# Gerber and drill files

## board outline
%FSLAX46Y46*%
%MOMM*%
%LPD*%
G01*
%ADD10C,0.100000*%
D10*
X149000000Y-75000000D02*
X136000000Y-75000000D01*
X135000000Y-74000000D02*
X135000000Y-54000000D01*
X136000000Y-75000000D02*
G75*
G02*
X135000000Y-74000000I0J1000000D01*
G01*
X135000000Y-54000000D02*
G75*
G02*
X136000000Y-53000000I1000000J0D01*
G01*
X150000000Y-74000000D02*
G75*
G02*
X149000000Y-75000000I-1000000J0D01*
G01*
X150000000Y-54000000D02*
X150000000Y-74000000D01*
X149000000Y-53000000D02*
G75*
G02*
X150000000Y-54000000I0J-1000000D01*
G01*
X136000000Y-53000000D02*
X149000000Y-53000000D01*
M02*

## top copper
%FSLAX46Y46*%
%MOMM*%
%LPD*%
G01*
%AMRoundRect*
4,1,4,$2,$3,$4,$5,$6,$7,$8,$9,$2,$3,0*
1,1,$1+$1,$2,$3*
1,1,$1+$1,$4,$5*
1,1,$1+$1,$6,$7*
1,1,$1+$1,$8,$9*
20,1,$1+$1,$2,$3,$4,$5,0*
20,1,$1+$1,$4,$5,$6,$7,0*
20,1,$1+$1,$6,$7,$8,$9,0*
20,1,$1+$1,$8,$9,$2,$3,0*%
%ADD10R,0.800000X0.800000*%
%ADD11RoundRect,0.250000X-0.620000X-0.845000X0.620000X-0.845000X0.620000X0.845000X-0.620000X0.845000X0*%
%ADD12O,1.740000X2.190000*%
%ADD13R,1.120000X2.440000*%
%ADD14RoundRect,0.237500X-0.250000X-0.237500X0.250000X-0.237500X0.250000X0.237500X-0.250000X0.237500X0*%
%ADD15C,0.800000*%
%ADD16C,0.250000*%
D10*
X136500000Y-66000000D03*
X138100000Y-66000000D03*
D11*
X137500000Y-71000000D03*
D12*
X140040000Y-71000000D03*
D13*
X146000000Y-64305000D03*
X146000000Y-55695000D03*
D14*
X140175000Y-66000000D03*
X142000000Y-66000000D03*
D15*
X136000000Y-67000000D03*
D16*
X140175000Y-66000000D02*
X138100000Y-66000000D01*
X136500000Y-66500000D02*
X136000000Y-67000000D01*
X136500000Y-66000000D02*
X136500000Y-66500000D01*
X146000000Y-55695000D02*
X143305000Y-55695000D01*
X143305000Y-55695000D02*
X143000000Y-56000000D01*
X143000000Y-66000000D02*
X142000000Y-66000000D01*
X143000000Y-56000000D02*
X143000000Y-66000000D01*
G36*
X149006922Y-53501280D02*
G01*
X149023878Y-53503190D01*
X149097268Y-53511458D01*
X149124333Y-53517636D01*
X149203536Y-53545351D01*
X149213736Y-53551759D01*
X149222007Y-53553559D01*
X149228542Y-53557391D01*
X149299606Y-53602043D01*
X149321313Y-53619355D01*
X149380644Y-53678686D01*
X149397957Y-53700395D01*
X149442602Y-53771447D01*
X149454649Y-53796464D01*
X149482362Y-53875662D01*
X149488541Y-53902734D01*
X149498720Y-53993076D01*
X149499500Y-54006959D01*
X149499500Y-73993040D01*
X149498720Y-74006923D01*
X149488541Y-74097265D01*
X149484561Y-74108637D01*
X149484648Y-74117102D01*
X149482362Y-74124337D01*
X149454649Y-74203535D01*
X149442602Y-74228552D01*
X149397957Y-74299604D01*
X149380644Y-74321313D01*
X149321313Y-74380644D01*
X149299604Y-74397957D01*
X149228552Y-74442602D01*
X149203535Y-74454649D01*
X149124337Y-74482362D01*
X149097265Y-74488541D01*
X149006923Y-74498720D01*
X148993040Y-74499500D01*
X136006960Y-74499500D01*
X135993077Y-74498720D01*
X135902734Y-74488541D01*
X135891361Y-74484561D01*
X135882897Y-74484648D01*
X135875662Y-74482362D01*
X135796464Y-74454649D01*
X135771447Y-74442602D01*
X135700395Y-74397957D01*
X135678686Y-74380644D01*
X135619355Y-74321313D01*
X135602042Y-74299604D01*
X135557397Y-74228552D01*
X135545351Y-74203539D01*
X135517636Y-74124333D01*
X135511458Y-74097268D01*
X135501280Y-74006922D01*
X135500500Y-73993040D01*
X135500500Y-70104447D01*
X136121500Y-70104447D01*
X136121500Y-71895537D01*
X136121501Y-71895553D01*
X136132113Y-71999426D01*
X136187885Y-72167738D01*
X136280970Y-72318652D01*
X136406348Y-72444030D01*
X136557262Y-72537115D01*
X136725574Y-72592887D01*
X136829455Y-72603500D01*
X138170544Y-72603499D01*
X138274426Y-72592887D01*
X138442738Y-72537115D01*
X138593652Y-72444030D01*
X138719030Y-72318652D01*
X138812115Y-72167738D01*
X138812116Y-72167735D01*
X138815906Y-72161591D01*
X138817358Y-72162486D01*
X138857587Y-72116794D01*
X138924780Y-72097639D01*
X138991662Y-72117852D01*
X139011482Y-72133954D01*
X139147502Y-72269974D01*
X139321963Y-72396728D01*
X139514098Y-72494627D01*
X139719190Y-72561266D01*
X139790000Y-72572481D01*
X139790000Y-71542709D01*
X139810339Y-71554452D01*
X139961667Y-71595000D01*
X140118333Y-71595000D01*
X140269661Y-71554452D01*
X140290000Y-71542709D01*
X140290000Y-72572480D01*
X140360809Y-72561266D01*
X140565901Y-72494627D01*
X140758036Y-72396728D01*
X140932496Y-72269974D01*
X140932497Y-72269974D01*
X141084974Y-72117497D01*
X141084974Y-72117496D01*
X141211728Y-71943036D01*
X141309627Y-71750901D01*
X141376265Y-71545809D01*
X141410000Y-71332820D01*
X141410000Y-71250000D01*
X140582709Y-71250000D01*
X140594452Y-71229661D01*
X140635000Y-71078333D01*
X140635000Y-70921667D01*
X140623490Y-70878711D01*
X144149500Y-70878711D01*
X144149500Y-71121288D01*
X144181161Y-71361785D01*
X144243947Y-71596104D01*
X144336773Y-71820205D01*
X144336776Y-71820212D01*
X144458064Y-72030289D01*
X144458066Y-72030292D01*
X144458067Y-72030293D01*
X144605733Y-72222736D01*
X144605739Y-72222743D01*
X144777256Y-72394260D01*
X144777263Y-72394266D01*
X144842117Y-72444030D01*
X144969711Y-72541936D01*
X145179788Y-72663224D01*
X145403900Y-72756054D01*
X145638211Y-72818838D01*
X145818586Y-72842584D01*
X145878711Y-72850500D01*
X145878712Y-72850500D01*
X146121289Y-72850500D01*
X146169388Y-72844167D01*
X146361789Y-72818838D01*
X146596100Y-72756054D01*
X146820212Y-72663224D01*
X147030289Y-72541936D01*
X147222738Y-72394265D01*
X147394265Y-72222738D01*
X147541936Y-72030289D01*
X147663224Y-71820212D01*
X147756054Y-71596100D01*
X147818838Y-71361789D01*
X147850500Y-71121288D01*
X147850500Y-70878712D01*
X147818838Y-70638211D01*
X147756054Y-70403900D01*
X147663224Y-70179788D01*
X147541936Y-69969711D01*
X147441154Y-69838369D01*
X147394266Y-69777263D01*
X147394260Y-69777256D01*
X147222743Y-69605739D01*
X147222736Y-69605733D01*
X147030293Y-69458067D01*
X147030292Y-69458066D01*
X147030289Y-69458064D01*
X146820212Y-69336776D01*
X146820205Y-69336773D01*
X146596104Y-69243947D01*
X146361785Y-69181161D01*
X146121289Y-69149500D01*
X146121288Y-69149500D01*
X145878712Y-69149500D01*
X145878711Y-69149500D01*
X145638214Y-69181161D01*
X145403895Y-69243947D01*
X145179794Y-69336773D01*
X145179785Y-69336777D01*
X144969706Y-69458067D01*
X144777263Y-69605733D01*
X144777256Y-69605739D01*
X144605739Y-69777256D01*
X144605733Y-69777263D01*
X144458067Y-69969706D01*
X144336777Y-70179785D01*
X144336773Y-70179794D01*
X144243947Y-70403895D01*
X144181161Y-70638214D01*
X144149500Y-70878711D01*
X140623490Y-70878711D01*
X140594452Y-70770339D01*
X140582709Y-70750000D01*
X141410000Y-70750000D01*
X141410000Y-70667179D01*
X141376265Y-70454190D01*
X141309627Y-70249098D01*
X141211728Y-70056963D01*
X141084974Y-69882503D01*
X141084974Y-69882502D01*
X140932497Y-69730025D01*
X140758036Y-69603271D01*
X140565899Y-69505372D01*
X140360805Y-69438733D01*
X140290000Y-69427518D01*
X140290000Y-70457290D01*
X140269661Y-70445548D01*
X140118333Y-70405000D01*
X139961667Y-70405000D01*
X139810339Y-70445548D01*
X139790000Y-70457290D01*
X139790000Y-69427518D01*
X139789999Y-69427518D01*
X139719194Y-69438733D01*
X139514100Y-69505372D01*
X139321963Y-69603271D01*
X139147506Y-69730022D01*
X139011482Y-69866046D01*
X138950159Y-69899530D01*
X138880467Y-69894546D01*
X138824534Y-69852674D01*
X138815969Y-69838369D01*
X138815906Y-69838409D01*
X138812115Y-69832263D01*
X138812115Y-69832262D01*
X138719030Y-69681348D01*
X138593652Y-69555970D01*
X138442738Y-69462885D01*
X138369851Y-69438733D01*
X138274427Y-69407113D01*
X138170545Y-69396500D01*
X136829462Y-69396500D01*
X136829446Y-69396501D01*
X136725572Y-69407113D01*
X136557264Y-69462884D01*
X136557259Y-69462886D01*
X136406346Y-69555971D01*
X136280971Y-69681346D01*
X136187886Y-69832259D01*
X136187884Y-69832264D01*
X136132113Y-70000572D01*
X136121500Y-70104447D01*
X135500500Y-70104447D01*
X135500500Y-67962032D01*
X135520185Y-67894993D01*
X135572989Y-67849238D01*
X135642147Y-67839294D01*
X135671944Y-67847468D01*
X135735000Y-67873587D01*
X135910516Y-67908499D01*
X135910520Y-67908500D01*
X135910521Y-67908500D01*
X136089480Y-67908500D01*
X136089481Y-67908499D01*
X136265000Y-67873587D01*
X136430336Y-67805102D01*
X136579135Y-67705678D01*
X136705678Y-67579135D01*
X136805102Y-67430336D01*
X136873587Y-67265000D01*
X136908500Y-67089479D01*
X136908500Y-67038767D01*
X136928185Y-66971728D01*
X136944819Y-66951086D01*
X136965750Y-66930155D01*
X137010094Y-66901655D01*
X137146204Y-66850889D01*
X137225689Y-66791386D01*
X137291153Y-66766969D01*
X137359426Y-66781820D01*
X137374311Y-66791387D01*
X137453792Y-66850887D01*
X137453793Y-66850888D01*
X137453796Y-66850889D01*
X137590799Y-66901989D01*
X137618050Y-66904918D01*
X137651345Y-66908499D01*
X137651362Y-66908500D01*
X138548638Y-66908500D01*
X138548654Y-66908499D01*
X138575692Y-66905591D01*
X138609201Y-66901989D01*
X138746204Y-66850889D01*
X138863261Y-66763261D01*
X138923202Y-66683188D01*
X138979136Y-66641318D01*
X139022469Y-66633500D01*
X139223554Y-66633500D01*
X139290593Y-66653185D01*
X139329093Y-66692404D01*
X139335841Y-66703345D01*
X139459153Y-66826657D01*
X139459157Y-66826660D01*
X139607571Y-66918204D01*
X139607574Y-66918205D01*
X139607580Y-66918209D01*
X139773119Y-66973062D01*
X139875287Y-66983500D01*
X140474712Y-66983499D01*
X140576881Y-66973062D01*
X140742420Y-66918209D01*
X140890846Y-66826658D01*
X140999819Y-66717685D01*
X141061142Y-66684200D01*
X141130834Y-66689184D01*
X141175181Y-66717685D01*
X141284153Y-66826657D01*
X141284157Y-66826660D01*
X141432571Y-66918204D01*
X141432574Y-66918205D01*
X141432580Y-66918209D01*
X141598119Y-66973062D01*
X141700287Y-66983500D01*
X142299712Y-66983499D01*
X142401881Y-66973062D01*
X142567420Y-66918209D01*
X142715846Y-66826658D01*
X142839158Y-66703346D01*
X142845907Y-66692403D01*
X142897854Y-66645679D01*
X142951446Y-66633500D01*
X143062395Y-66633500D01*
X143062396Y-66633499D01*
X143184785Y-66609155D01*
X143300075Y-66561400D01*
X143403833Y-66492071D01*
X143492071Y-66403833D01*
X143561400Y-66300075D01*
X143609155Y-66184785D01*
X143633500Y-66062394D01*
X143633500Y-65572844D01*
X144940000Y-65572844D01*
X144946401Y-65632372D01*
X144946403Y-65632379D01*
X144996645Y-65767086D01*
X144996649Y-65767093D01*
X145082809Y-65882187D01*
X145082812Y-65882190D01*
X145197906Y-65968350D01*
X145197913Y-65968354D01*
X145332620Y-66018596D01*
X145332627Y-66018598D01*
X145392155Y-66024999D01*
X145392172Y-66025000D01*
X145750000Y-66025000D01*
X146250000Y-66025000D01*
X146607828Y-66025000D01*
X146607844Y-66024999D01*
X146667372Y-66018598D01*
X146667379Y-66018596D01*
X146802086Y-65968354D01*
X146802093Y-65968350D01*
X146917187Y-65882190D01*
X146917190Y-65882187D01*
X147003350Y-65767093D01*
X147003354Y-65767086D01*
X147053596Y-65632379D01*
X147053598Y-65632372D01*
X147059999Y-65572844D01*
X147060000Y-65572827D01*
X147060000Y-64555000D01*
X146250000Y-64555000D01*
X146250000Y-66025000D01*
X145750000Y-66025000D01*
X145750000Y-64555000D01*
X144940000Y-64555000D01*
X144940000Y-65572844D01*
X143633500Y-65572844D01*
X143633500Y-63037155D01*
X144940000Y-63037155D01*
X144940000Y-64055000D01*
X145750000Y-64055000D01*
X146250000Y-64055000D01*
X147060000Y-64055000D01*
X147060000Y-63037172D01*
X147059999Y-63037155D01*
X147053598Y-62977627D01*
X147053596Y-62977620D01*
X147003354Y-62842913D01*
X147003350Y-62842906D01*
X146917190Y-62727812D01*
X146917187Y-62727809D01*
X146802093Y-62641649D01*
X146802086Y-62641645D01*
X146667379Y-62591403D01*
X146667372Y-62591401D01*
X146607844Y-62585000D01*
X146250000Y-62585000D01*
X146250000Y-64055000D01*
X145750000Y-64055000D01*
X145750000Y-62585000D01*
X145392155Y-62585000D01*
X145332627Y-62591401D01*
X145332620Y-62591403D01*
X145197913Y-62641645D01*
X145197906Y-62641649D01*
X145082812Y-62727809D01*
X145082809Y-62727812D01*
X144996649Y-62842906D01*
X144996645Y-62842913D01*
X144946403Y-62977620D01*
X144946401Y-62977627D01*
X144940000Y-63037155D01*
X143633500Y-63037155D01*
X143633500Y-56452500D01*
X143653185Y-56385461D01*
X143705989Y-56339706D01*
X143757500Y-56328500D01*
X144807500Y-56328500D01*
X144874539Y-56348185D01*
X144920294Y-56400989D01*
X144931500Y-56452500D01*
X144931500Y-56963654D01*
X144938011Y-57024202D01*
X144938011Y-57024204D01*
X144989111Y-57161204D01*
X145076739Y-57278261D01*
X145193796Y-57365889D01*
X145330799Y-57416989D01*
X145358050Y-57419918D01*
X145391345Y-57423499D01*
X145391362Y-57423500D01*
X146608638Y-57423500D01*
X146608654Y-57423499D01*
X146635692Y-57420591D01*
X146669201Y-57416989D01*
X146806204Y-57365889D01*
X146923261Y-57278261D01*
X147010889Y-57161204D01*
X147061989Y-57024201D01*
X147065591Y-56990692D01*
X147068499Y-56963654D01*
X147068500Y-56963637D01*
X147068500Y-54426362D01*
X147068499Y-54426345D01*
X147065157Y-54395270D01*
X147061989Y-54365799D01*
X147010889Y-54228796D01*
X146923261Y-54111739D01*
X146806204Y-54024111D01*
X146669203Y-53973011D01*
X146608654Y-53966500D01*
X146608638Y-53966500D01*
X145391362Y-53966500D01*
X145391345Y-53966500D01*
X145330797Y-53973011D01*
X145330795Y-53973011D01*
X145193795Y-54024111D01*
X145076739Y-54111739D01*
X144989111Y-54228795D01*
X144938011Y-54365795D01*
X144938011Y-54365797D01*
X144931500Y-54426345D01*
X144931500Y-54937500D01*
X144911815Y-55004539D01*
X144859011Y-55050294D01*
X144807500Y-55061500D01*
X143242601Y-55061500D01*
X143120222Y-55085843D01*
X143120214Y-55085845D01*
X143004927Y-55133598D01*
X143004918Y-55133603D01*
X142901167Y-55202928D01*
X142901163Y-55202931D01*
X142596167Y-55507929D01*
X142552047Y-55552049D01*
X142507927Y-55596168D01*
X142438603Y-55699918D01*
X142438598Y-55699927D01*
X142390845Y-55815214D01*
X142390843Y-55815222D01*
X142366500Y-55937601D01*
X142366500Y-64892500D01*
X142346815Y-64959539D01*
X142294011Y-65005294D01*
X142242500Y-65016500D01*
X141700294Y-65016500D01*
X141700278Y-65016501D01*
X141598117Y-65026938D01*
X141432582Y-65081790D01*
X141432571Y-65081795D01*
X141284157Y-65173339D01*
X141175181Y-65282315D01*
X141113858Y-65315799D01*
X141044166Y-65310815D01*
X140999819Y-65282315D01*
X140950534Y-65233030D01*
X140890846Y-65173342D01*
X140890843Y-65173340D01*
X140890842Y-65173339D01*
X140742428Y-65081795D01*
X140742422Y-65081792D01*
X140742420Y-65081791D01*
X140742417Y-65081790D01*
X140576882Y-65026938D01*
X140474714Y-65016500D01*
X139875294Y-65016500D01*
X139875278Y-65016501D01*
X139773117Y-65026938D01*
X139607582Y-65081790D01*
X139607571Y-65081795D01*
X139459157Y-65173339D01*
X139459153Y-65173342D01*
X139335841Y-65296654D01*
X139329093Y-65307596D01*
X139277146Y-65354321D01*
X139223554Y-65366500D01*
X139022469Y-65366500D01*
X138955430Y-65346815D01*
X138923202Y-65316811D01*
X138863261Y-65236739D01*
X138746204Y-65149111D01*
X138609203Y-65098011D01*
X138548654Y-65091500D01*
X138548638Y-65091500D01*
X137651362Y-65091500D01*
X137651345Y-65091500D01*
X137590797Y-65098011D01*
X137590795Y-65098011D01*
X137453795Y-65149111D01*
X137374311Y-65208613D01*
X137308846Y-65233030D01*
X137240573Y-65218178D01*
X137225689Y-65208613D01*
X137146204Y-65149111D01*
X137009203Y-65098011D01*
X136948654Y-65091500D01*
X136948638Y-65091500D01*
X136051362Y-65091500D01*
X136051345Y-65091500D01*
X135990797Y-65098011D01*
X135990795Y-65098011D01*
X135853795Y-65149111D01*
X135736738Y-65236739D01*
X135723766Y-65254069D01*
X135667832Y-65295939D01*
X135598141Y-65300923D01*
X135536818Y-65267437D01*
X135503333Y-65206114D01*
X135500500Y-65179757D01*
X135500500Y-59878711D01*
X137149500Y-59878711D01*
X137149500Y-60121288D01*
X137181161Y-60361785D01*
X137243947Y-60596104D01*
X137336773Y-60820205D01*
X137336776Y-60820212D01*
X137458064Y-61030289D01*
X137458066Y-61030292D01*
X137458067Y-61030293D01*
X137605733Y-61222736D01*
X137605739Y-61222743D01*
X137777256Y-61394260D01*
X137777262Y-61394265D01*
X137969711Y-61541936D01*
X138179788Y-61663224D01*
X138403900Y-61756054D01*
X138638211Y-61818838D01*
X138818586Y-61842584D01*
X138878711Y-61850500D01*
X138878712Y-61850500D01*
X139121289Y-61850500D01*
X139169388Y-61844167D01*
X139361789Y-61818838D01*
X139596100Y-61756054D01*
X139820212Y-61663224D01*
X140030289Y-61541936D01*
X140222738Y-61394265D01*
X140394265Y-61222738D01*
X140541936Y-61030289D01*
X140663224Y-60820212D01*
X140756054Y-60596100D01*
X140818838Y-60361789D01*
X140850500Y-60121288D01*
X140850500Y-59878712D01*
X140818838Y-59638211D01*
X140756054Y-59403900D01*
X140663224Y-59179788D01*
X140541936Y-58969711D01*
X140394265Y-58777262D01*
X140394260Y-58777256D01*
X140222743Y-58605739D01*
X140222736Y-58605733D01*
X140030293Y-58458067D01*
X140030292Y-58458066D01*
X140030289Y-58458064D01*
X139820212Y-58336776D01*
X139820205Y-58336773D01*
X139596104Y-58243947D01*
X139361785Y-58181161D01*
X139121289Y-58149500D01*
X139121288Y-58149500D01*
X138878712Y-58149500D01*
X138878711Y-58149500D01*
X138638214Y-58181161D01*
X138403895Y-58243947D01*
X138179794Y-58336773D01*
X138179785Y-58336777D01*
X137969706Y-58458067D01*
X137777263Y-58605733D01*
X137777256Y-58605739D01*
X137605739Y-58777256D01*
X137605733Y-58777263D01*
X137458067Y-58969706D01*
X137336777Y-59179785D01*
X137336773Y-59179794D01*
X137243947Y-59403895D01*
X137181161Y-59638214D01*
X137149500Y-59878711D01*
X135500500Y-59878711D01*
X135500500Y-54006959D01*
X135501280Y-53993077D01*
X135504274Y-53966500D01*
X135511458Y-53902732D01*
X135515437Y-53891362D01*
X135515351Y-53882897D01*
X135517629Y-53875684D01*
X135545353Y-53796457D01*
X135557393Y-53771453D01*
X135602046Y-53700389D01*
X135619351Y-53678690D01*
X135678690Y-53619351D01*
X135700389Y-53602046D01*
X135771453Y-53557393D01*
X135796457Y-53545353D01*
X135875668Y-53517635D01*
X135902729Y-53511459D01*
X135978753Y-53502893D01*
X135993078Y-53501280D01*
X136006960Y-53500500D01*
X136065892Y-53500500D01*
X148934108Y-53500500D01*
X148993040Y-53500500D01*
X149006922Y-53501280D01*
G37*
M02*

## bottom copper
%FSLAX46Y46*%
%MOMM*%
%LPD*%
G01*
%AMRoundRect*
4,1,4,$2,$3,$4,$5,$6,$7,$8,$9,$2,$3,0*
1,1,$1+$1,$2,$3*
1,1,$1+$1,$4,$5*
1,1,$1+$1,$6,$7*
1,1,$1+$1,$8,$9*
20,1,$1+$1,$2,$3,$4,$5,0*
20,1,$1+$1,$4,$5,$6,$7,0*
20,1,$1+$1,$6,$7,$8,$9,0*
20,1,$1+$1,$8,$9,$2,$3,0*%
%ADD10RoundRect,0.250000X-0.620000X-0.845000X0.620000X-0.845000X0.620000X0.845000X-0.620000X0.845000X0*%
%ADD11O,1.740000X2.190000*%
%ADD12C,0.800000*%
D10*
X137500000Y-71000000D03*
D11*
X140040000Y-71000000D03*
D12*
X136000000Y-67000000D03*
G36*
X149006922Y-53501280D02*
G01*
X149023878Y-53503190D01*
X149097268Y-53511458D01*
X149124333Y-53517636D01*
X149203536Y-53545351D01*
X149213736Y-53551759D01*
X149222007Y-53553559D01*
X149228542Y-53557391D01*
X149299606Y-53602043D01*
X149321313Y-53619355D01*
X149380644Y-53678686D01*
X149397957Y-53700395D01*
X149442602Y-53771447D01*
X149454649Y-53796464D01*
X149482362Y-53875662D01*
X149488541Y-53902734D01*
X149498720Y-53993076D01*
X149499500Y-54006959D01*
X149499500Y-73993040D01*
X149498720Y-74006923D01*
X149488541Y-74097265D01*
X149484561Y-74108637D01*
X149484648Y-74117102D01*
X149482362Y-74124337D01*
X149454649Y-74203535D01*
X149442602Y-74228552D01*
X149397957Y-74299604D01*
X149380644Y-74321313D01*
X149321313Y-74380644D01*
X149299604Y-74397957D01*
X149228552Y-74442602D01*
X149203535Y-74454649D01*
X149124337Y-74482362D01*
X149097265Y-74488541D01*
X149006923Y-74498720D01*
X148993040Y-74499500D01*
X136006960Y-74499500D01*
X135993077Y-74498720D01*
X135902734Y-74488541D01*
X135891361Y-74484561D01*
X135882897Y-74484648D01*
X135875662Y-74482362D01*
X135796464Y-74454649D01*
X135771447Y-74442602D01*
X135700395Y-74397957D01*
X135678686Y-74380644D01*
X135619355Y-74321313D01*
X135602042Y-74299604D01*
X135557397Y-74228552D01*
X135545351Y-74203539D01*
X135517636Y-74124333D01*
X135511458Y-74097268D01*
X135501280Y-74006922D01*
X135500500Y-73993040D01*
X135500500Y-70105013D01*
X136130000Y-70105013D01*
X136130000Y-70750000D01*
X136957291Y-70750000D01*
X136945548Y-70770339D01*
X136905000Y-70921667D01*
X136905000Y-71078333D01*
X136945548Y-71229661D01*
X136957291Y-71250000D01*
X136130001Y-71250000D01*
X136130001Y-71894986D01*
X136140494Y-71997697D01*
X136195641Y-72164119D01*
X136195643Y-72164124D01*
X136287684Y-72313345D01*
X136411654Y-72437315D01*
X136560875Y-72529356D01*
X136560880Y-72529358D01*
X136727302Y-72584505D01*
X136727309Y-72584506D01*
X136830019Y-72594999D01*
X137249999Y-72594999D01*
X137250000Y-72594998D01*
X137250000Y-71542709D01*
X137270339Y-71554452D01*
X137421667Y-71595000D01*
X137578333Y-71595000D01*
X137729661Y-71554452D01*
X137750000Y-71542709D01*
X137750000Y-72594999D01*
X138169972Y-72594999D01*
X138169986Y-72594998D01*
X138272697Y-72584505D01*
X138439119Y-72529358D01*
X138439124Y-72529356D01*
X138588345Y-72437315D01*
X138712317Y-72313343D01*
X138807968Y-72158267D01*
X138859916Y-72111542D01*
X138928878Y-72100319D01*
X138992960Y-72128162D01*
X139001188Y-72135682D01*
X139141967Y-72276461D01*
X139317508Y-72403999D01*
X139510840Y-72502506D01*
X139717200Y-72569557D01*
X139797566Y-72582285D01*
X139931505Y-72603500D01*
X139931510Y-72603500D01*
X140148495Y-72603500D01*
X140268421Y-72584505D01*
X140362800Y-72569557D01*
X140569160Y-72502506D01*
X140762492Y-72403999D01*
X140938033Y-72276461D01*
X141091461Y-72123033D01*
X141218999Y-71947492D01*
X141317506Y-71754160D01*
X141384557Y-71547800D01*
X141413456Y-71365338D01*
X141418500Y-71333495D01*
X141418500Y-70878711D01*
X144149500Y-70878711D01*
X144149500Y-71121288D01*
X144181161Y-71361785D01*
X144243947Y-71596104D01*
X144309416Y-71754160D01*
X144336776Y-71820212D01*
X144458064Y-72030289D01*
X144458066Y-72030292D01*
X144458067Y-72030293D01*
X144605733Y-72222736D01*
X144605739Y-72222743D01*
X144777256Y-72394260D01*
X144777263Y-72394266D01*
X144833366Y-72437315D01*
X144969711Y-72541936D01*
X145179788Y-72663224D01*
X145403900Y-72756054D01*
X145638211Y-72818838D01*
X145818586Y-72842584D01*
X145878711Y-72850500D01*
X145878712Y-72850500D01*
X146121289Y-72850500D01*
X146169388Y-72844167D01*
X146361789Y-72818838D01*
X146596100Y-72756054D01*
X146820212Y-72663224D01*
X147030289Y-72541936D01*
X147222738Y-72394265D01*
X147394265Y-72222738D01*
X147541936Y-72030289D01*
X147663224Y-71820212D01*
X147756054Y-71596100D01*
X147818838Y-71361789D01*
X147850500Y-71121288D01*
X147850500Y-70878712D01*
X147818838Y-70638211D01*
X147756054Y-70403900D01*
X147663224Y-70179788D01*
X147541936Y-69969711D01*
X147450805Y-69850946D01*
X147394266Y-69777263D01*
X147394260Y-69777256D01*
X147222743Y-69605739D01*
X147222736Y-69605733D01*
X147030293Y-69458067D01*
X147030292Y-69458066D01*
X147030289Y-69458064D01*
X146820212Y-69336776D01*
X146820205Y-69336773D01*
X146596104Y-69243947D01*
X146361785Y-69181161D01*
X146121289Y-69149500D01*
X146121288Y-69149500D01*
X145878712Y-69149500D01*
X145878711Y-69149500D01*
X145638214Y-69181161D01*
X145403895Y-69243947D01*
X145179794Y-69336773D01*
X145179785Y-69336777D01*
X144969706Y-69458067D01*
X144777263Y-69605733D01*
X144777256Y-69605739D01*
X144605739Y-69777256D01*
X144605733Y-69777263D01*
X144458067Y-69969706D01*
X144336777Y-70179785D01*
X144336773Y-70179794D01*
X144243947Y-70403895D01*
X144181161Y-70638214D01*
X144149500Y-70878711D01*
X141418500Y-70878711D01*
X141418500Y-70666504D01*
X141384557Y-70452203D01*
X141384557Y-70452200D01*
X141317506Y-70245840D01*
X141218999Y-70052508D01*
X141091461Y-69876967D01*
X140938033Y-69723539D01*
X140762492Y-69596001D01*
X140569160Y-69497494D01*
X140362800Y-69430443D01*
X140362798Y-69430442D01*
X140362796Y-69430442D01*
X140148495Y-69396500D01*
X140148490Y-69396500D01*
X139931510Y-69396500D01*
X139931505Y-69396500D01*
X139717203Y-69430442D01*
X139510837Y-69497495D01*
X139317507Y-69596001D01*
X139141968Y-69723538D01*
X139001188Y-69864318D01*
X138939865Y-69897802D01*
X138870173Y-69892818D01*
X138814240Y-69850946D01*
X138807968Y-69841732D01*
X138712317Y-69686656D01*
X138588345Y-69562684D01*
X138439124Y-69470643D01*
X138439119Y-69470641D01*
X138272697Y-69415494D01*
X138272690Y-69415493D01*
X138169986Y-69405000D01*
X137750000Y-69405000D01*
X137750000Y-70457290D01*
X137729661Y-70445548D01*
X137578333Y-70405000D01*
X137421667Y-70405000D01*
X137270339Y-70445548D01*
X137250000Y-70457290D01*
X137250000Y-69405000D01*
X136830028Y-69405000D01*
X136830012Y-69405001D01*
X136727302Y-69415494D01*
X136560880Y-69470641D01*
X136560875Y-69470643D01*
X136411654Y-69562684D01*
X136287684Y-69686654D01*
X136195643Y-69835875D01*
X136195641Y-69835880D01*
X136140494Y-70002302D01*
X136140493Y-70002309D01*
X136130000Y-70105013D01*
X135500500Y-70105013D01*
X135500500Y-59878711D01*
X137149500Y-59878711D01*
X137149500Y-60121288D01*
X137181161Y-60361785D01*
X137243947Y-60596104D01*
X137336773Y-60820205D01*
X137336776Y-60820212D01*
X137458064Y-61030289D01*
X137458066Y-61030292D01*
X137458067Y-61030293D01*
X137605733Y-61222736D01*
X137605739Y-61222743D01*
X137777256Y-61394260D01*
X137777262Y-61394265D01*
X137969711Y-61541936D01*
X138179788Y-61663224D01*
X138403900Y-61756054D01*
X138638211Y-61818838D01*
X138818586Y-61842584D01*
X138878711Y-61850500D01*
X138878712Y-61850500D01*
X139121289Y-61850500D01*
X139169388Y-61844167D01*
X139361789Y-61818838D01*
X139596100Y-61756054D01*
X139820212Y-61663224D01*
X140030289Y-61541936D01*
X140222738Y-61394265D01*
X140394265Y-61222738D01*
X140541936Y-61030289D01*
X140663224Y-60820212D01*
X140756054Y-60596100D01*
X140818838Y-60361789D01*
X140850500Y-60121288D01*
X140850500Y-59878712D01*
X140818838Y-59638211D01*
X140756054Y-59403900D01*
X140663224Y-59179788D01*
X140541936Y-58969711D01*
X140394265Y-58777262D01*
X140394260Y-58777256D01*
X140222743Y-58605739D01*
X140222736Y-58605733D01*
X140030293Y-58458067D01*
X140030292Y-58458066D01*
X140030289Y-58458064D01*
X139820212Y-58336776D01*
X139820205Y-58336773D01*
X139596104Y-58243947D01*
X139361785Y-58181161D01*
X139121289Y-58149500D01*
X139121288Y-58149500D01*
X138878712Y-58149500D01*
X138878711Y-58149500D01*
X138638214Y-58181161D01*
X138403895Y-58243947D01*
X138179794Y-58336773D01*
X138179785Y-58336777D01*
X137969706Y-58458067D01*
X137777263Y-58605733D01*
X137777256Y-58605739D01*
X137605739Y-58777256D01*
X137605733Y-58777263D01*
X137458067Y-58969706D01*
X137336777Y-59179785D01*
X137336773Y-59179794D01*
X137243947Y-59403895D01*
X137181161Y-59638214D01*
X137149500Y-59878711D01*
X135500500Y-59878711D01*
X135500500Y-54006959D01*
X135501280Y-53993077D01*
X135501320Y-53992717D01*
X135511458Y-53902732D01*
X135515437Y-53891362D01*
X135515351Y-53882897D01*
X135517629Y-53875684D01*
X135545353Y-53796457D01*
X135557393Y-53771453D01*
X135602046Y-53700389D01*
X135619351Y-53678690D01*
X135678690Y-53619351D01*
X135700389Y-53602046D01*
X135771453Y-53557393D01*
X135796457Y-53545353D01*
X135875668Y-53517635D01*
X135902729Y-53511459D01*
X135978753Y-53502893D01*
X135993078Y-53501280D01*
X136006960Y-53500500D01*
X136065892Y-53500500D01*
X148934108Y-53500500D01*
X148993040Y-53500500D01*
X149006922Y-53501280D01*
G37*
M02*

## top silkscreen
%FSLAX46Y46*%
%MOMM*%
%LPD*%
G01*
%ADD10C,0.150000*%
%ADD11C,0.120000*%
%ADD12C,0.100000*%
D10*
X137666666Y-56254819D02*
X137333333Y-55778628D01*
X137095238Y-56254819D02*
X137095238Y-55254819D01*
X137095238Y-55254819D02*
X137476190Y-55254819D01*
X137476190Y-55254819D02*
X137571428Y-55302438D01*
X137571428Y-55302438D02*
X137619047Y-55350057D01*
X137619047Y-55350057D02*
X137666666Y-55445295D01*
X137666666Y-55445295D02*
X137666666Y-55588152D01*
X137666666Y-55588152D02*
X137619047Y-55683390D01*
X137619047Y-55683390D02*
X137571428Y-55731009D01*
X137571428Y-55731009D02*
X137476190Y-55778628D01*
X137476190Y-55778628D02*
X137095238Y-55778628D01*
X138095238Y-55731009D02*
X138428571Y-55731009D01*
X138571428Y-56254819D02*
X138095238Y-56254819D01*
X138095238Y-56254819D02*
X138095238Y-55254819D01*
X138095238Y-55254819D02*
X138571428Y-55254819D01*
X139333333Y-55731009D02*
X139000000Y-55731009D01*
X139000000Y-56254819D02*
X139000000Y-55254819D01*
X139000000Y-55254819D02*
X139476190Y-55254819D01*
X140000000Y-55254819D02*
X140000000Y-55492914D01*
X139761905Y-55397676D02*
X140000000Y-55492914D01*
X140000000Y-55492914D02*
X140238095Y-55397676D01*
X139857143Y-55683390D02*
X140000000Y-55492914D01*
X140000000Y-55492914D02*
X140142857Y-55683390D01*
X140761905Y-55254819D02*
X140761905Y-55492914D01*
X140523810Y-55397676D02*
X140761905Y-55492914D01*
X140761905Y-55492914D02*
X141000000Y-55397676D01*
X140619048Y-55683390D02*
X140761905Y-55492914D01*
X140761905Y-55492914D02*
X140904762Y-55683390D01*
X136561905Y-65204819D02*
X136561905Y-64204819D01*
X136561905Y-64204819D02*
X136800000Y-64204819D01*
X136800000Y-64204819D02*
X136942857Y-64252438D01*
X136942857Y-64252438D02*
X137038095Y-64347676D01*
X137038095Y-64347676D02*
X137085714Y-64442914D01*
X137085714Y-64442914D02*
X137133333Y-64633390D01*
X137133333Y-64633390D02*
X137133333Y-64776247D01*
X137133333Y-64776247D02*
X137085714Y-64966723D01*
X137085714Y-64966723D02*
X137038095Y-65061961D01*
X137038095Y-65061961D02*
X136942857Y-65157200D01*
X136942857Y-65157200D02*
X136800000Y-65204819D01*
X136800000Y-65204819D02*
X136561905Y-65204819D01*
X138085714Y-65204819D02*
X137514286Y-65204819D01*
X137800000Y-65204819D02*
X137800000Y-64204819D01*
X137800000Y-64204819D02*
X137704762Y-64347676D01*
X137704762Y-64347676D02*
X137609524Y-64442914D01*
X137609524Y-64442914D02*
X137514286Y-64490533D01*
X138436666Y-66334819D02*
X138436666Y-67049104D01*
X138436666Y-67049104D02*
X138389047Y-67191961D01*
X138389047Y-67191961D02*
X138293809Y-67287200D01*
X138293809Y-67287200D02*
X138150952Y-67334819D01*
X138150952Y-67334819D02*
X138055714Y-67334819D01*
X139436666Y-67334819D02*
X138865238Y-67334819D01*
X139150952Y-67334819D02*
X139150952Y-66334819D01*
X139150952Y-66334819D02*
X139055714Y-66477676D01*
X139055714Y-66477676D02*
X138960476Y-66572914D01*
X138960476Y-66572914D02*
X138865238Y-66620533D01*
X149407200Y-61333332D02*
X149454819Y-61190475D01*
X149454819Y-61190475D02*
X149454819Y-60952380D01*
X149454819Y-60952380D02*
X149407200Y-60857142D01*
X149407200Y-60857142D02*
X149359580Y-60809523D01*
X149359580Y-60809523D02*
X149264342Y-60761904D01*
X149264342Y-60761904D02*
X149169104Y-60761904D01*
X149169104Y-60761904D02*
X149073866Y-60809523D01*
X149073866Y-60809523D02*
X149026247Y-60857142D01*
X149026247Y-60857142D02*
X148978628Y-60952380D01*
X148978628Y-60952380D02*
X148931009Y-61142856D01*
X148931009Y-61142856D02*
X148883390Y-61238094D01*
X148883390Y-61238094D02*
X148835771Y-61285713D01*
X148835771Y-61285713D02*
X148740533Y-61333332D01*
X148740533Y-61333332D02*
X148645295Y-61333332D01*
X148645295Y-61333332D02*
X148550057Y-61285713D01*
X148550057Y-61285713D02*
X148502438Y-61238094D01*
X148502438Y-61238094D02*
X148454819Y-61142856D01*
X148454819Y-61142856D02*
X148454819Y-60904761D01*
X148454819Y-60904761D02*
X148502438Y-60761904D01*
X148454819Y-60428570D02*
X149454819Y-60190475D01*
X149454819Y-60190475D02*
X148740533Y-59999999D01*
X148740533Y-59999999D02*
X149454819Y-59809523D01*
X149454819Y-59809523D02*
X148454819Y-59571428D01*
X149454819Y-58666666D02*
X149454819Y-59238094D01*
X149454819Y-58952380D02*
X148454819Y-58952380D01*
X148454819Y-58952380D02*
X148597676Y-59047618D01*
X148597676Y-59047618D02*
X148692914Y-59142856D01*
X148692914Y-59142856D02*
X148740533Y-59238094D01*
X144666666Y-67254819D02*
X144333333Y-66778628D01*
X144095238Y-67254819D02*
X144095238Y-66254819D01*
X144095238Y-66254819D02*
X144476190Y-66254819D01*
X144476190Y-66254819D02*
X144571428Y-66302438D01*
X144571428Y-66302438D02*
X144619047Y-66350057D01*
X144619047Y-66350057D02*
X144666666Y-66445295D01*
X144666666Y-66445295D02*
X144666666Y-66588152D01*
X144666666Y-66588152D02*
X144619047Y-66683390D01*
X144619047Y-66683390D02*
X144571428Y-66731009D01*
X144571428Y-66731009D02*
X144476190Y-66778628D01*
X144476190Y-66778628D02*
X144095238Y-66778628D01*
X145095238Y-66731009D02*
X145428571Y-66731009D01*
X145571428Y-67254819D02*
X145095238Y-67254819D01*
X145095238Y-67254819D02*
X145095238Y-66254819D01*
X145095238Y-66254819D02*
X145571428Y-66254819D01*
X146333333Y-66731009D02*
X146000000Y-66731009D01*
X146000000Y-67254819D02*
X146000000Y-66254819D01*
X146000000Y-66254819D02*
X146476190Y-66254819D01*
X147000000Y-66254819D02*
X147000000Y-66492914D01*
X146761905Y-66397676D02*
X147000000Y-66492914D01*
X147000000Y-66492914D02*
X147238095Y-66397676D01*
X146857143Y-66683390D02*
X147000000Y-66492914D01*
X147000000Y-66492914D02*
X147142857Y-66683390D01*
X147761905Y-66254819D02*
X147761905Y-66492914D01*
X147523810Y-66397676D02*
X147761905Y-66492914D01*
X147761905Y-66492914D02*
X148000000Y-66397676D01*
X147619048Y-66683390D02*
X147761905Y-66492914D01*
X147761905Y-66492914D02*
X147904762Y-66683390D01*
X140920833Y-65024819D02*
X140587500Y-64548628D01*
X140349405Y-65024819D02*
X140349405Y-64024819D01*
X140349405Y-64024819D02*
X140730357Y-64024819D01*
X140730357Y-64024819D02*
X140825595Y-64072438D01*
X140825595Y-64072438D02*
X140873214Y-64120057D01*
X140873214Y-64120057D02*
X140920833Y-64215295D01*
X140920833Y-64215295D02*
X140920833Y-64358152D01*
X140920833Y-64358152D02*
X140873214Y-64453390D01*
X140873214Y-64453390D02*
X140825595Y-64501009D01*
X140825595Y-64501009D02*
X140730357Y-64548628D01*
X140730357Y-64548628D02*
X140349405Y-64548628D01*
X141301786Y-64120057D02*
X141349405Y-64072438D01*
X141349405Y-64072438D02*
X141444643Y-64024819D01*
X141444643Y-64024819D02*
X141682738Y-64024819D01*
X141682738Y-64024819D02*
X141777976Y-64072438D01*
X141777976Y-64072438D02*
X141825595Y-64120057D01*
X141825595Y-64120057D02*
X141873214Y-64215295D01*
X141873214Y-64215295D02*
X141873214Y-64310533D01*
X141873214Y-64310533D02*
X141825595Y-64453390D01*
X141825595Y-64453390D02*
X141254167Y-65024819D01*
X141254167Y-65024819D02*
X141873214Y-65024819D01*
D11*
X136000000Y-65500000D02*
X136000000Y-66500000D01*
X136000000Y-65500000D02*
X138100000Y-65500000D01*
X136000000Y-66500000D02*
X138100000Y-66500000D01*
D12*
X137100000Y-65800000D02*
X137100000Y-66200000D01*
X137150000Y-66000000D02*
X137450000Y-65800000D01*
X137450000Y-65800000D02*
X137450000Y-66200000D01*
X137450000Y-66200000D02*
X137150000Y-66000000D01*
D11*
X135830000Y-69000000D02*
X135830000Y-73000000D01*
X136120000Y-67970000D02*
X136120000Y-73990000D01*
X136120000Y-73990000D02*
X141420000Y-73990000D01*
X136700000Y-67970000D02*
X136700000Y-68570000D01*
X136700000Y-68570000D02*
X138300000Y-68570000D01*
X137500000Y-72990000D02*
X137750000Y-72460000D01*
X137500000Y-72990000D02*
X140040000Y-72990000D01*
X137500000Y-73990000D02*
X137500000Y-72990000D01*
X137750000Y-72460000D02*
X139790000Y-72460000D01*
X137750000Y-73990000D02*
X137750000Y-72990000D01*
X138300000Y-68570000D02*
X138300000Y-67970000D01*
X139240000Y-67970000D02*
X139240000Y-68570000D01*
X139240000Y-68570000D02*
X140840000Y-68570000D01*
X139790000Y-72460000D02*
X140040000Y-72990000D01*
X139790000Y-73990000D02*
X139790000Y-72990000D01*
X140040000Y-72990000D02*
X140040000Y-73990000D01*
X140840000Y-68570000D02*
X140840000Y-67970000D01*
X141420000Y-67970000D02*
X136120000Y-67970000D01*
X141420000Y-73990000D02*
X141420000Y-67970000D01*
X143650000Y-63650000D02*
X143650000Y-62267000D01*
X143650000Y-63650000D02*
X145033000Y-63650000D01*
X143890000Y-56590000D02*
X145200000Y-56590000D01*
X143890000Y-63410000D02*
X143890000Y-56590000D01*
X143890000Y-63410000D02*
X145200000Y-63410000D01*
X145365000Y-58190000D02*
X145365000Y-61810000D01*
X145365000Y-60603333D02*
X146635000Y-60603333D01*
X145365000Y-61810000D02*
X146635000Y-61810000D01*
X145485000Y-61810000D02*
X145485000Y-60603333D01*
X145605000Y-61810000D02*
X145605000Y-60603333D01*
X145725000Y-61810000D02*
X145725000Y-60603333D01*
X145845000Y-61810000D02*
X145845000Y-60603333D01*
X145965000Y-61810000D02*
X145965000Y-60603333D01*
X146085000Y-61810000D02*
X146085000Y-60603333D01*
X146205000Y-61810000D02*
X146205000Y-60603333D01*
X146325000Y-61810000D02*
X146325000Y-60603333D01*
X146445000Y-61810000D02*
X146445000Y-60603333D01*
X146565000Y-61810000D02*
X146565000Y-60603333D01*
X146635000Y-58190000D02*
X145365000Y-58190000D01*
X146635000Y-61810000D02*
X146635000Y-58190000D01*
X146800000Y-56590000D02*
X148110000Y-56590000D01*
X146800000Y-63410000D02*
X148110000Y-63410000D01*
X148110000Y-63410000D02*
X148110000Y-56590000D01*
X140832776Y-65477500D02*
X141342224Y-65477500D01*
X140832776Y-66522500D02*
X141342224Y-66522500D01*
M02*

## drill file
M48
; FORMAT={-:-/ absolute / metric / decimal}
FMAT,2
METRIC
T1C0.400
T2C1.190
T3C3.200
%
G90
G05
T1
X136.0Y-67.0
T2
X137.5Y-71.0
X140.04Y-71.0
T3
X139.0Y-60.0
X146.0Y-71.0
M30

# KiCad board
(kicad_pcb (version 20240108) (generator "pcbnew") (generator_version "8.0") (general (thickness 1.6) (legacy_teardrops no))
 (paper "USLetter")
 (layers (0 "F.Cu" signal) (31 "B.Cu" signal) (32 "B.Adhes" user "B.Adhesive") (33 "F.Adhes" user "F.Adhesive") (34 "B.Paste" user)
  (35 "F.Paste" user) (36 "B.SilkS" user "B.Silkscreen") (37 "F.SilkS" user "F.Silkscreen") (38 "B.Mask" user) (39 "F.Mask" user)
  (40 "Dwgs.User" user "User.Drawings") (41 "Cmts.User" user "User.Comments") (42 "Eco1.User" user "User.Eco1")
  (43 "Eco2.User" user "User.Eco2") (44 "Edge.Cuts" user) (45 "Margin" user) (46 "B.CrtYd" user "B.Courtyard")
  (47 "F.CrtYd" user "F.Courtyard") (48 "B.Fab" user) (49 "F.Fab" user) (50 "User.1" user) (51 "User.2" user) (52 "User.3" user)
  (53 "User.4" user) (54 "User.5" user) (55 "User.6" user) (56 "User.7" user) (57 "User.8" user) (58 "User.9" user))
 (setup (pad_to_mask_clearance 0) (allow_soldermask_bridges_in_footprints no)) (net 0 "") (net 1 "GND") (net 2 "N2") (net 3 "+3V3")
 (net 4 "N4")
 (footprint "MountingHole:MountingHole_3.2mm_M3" (layer "F.Cu") (at 139 60)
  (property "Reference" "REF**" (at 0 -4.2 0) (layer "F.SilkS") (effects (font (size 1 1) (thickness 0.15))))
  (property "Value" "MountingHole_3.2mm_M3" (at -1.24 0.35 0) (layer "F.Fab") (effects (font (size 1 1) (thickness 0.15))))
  (pad "" np_thru_hole circle (at 0 0) (size 3.2 3.2) (drill 3.2) (layers "*.Cu" "*.Mask")))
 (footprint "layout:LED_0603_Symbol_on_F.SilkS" (layer "F.Cu") (at 137.3 66)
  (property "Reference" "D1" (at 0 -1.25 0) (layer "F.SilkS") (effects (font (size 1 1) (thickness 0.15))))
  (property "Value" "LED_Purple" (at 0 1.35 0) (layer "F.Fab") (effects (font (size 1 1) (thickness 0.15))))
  (fp_line (start -1.3 -0.5) (end -1.3 0.5) (stroke (width 0.12) (type solid)) (layer "F.SilkS"))
  (fp_line (start -1.3 -0.5) (end 0.8 -0.5) (stroke (width 0.12) (type solid)) (layer "F.SilkS"))
  (fp_line (start -1.3 0.5) (end 0.8 0.5) (stroke (width 0.12) (type solid)) (layer "F.SilkS"))
  (fp_line (start -0.2 -0.2) (end -0.2 0.2) (stroke (width 0.1) (type solid)) (layer "F.SilkS"))
  (fp_line (start -0.15 0) (end 0.15 -0.2) (stroke (width 0.1) (type solid)) (layer "F.SilkS"))
  (fp_line (start 0.15 -0.2) (end 0.15 0.2) (stroke (width 0.1) (type solid)) (layer "F.SilkS"))
  (fp_line (start 0.15 0.2) (end -0.15 0) (stroke (width 0.1) (type solid)) (layer "F.SilkS"))
  (pad "1" smd rect (at -0.8 0 180) (size 0.8 0.8) (layers "F.Cu" "F.Paste" "F.Mask") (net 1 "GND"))
  (pad "2" smd rect (at 0.8 0 180) (size 0.8 0.8) (layers "F.Cu" "F.Paste" "F.Mask") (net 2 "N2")))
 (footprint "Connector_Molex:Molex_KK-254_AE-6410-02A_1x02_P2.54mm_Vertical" (layer "F.Cu") (at 137.5 71)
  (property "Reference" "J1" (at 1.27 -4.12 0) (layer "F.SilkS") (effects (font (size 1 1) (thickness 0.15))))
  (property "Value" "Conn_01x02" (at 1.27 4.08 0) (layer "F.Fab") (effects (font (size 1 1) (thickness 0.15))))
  (fp_line (start -1.67 -2) (end -1.67 2) (stroke (width 0.12) (type solid)) (layer "F.SilkS"))
  (fp_line (start -1.38 -3.03) (end -1.38 2.99) (stroke (width 0.12) (type solid)) (layer "F.SilkS"))
  (fp_line (start -1.38 2.99) (end 3.92 2.99) (stroke (width 0.12) (type solid)) (layer "F.SilkS"))
  (fp_line (start -0.8 -3.03) (end -0.8 -2.43) (stroke (width 0.12) (type solid)) (layer "F.SilkS"))
  (fp_line (start -0.8 -2.43) (end 0.8 -2.43) (stroke (width 0.12) (type solid)) (layer "F.SilkS"))
  (fp_line (start 0 1.99) (end 0.25 1.46) (stroke (width 0.12) (type solid)) (layer "F.SilkS"))
  (fp_line (start 0 1.99) (end 2.54 1.99) (stroke (width 0.12) (type solid)) (layer "F.SilkS"))
  (fp_line (start 0 2.99) (end 0 1.99) (stroke (width 0.12) (type solid)) (layer "F.SilkS"))
  (fp_line (start 0.25 1.46) (end 2.29 1.46) (stroke (width 0.12) (type solid)) (layer "F.SilkS"))
  (fp_line (start 0.25 2.99) (end 0.25 1.99) (stroke (width 0.12) (type solid)) (layer "F.SilkS"))
  (fp_line (start 0.8 -2.43) (end 0.8 -3.03) (stroke (width 0.12) (type solid)) (layer "F.SilkS"))
  (fp_line (start 1.74 -3.03) (end 1.74 -2.43) (stroke (width 0.12) (type solid)) (layer "F.SilkS"))
  (fp_line (start 1.74 -2.43) (end 3.34 -2.43) (stroke (width 0.12) (type solid)) (layer "F.SilkS"))
  (fp_line (start 2.29 1.46) (end 2.54 1.99) (stroke (width 0.12) (type solid)) (layer "F.SilkS"))
  (fp_line (start 2.29 2.99) (end 2.29 1.99) (stroke (width 0.12) (type solid)) (layer "F.SilkS"))
  (fp_line (start 2.54 1.99) (end 2.54 2.99) (stroke (width 0.12) (type solid)) (layer "F.SilkS"))
  (fp_line (start 3.34 -2.43) (end 3.34 -3.03) (stroke (width 0.12) (type solid)) (layer "F.SilkS"))
  (fp_line (start 3.92 -3.03) (end -1.38 -3.03) (stroke (width 0.12) (type solid)) (layer "F.SilkS"))
  (fp_line (start 3.92 2.99) (end 3.92 -3.03) (stroke (width 0.12) (type solid)) (layer "F.SilkS"))
  (pad "1" thru_hole roundrect (at 0 0) (size 1.74 2.19) (drill 1.19) (layers "*.Cu" "*.Mask") (remove_unused_layers no)
   (roundrect_rratio 0.143678) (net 1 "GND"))
  (pad "2" thru_hole oval (at 2.54 0) (size 1.74 2.19) (drill 1.19) (layers "*.Cu" "*.Mask") (remove_unused_layers no) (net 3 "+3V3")))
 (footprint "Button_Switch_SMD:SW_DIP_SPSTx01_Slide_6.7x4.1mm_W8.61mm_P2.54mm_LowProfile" (layer "F.Cu") (at 146 60 90)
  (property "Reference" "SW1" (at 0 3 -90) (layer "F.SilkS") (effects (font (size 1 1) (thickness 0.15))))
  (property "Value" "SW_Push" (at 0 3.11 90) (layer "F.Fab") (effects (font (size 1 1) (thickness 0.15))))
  (fp_line (start -3.65 -2.35) (end -2.267 -2.35) (stroke (width 0.12) (type solid)) (layer "F.SilkS"))
  (fp_line (start -3.65 -2.35) (end -3.65 -0.967) (stroke (width 0.12) (type solid)) (layer "F.SilkS"))
  (fp_line (start 3.41 -2.11) (end 3.41 -0.8) (stroke (width 0.12) (type solid)) (layer "F.SilkS"))
  (fp_line (start -3.41 -2.11) (end 3.41 -2.11) (stroke (width 0.12) (type solid)) (layer "F.SilkS"))
  (fp_line (start -3.41 -2.11) (end -3.41 -0.8) (stroke (width 0.12) (type solid)) (layer "F.SilkS"))
  (fp_line (start 1.81 -0.635) (end -1.81 -0.635) (stroke (width 0.12) (type solid)) (layer "F.SilkS"))
  (fp_line (start -0.603333 -0.635) (end -0.603333 0.635) (stroke (width 0.12) (type solid)) (layer "F.SilkS"))
  (fp_line (start -1.81 -0.635) (end -1.81 0.635) (stroke (width 0.12) (type solid)) (layer "F.SilkS"))
  (fp_line (start -1.81 -0.515) (end -0.603333 -0.515) (stroke (width 0.12) (type solid)) (layer "F.SilkS"))
  (fp_line (start -1.81 -0.395) (end -0.603333 -0.395) (stroke (width 0.12) (type solid)) (layer "F.SilkS"))
  (fp_line (start -1.81 -0.275) (end -0.603333 -0.275) (stroke (width 0.12) (type solid)) (layer "F.SilkS"))
  (fp_line (start -1.81 -0.155) (end -0.603333 -0.155) (stroke (width 0.12) (type solid)) (layer "F.SilkS"))
  (fp_line (start -1.81 -0.035) (end -0.603333 -0.035) (stroke (width 0.12) (type solid)) (layer "F.SilkS"))
  (fp_line (start -1.81 0.085) (end -0.603333 0.085) (stroke (width 0.12) (type solid)) (layer "F.SilkS"))
  (fp_line (start -1.81 0.205) (end -0.603333 0.205) (stroke (width 0.12) (type solid)) (layer "F.SilkS"))
  (fp_line (start -1.81 0.325) (end -0.603333 0.325) (stroke (width 0.12) (type solid)) (layer "F.SilkS"))
  (fp_line (start -1.81 0.445) (end -0.603333 0.445) (stroke (width 0.12) (type solid)) (layer "F.SilkS"))
  (fp_line (start -1.81 0.565) (end -0.603333 0.565) (stroke (width 0.12) (type solid)) (layer "F.SilkS"))
  (fp_line (start 1.81 0.635) (end 1.81 -0.635) (stroke (width 0.12) (type solid)) (layer "F.SilkS"))
  (fp_line (start -1.81 0.635) (end 1.81 0.635) (stroke (width 0.12) (type solid)) (layer "F.SilkS"))
  (fp_line (start 3.41 0.8) (end 3.41 2.11) (stroke (width 0.12) (type solid)) (layer "F.SilkS"))
  (fp_line (start -3.41 0.8) (end -3.41 2.11) (stroke (width 0.12) (type solid)) (layer "F.SilkS"))
  (fp_line (start -3.41 2.11) (end 3.41 2.11) (stroke (width 0.12) (type solid)) (layer "F.SilkS"))
  (pad "1" smd rect (at -4.305 0 90) (size 2.44 1.12) (layers "F.Cu" "F.Paste" "F.Mask") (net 3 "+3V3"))
  (pad "2" smd rect (at 4.305 0 90) (size 2.44 1.12) (layers "F.Cu" "F.Paste" "F.Mask") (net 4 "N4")))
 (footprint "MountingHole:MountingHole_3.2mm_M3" (layer "F.Cu") (at 146 71)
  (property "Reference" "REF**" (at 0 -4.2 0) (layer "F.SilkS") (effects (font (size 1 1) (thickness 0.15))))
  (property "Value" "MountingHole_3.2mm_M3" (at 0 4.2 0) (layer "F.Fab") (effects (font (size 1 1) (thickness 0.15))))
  (pad "" np_thru_hole circle (at 0 0) (size 3.2 3.2) (drill 3.2) (layers "*.Cu" "*.Mask")))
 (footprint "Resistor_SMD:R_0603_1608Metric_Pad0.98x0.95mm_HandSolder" (layer "F.Cu") (at 141.0875 66)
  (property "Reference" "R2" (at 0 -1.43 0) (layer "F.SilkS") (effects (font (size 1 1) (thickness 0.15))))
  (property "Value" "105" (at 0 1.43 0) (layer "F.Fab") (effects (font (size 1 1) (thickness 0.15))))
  (fp_line (start -0.254724 -0.5225) (end 0.254724 -0.5225) (stroke (width 0.12) (type solid)) (layer "F.SilkS"))
  (fp_line (start -0.254724 0.5225) (end 0.254724 0.5225) (stroke (width 0.12) (type solid)) (layer "F.SilkS"))
  (pad "1" smd roundrect (at -0.9125 0) (size 0.975 0.95) (layers "F.Cu" "F.Paste" "F.Mask") (roundrect_rratio 0.25) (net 2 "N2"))
  (pad "2" smd roundrect (at 0.9125 0) (size 0.975 0.95) (layers "F.Cu" "F.Paste" "F.Mask") (roundrect_rratio 0.25) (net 4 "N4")))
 (gr_line (start 149 75) (end 136 75) (stroke (width 0.1) (type default)) (layer "Edge.Cuts"))
 (gr_line (start 135 74) (end 135 54) (stroke (width 0.1) (type default)) (layer "Edge.Cuts"))
 (gr_arc (start 136 75) (mid 135.292893 74.707107) (end 135 74) (stroke (width 0.1) (type default)) (layer "Edge.Cuts"))
 (gr_arc (start 135 54) (mid 135.292893 53.292893) (end 136 53) (stroke (width 0.1) (type default)) (layer "Edge.Cuts"))
 (gr_arc (start 150 74) (mid 149.707107 74.707107) (end 149 75) (stroke (width 0.1) (type default)) (layer "Edge.Cuts"))
 (gr_line (start 150 54) (end 150 74) (stroke (width 0.1) (type default)) (layer "Edge.Cuts"))
 (gr_arc (start 149 53) (mid 149.707107 53.292893) (end 150 54) (stroke (width 0.1) (type default)) (layer "Edge.Cuts"))
 (gr_line (start 136 53) (end 149 53) (stroke (width 0.1) (type default)) (layer "Edge.Cuts"))
 (segment (start 140.175 66) (end 138.1 66) (width 0.25) (layer "F.Cu") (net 2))
 (segment (start 136.5 66.5) (end 136 67) (width 0.25) (layer "F.Cu") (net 1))
 (segment (start 136.5 66) (end 136.5 66.5) (width 0.25) (layer "F.Cu") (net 1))
 (via (at 136 67) (size 0.8) (drill 0.4) (layers "F.Cu" "B.Cu") (free yes) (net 1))
 (segment (start 146 55.695) (end 143.305 55.695) (width 0.25) (layer "F.Cu") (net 4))
 (segment (start 143.305 55.695) (end 143 56) (width 0.25) (layer "F.Cu") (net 4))
 (segment (start 143 66) (end 142 66) (width 0.25) (layer "F.Cu") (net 4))
 (segment (start 143 56) (end 143 66) (width 0.25) (layer "F.Cu") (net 4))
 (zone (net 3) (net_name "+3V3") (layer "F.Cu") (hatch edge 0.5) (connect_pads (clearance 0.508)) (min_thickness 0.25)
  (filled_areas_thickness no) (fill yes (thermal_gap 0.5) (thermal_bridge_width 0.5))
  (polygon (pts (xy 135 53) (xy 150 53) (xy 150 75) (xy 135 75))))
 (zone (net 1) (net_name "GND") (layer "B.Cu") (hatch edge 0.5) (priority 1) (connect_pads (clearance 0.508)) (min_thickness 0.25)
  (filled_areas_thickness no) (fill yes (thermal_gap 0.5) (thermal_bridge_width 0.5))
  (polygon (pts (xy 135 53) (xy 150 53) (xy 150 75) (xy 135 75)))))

